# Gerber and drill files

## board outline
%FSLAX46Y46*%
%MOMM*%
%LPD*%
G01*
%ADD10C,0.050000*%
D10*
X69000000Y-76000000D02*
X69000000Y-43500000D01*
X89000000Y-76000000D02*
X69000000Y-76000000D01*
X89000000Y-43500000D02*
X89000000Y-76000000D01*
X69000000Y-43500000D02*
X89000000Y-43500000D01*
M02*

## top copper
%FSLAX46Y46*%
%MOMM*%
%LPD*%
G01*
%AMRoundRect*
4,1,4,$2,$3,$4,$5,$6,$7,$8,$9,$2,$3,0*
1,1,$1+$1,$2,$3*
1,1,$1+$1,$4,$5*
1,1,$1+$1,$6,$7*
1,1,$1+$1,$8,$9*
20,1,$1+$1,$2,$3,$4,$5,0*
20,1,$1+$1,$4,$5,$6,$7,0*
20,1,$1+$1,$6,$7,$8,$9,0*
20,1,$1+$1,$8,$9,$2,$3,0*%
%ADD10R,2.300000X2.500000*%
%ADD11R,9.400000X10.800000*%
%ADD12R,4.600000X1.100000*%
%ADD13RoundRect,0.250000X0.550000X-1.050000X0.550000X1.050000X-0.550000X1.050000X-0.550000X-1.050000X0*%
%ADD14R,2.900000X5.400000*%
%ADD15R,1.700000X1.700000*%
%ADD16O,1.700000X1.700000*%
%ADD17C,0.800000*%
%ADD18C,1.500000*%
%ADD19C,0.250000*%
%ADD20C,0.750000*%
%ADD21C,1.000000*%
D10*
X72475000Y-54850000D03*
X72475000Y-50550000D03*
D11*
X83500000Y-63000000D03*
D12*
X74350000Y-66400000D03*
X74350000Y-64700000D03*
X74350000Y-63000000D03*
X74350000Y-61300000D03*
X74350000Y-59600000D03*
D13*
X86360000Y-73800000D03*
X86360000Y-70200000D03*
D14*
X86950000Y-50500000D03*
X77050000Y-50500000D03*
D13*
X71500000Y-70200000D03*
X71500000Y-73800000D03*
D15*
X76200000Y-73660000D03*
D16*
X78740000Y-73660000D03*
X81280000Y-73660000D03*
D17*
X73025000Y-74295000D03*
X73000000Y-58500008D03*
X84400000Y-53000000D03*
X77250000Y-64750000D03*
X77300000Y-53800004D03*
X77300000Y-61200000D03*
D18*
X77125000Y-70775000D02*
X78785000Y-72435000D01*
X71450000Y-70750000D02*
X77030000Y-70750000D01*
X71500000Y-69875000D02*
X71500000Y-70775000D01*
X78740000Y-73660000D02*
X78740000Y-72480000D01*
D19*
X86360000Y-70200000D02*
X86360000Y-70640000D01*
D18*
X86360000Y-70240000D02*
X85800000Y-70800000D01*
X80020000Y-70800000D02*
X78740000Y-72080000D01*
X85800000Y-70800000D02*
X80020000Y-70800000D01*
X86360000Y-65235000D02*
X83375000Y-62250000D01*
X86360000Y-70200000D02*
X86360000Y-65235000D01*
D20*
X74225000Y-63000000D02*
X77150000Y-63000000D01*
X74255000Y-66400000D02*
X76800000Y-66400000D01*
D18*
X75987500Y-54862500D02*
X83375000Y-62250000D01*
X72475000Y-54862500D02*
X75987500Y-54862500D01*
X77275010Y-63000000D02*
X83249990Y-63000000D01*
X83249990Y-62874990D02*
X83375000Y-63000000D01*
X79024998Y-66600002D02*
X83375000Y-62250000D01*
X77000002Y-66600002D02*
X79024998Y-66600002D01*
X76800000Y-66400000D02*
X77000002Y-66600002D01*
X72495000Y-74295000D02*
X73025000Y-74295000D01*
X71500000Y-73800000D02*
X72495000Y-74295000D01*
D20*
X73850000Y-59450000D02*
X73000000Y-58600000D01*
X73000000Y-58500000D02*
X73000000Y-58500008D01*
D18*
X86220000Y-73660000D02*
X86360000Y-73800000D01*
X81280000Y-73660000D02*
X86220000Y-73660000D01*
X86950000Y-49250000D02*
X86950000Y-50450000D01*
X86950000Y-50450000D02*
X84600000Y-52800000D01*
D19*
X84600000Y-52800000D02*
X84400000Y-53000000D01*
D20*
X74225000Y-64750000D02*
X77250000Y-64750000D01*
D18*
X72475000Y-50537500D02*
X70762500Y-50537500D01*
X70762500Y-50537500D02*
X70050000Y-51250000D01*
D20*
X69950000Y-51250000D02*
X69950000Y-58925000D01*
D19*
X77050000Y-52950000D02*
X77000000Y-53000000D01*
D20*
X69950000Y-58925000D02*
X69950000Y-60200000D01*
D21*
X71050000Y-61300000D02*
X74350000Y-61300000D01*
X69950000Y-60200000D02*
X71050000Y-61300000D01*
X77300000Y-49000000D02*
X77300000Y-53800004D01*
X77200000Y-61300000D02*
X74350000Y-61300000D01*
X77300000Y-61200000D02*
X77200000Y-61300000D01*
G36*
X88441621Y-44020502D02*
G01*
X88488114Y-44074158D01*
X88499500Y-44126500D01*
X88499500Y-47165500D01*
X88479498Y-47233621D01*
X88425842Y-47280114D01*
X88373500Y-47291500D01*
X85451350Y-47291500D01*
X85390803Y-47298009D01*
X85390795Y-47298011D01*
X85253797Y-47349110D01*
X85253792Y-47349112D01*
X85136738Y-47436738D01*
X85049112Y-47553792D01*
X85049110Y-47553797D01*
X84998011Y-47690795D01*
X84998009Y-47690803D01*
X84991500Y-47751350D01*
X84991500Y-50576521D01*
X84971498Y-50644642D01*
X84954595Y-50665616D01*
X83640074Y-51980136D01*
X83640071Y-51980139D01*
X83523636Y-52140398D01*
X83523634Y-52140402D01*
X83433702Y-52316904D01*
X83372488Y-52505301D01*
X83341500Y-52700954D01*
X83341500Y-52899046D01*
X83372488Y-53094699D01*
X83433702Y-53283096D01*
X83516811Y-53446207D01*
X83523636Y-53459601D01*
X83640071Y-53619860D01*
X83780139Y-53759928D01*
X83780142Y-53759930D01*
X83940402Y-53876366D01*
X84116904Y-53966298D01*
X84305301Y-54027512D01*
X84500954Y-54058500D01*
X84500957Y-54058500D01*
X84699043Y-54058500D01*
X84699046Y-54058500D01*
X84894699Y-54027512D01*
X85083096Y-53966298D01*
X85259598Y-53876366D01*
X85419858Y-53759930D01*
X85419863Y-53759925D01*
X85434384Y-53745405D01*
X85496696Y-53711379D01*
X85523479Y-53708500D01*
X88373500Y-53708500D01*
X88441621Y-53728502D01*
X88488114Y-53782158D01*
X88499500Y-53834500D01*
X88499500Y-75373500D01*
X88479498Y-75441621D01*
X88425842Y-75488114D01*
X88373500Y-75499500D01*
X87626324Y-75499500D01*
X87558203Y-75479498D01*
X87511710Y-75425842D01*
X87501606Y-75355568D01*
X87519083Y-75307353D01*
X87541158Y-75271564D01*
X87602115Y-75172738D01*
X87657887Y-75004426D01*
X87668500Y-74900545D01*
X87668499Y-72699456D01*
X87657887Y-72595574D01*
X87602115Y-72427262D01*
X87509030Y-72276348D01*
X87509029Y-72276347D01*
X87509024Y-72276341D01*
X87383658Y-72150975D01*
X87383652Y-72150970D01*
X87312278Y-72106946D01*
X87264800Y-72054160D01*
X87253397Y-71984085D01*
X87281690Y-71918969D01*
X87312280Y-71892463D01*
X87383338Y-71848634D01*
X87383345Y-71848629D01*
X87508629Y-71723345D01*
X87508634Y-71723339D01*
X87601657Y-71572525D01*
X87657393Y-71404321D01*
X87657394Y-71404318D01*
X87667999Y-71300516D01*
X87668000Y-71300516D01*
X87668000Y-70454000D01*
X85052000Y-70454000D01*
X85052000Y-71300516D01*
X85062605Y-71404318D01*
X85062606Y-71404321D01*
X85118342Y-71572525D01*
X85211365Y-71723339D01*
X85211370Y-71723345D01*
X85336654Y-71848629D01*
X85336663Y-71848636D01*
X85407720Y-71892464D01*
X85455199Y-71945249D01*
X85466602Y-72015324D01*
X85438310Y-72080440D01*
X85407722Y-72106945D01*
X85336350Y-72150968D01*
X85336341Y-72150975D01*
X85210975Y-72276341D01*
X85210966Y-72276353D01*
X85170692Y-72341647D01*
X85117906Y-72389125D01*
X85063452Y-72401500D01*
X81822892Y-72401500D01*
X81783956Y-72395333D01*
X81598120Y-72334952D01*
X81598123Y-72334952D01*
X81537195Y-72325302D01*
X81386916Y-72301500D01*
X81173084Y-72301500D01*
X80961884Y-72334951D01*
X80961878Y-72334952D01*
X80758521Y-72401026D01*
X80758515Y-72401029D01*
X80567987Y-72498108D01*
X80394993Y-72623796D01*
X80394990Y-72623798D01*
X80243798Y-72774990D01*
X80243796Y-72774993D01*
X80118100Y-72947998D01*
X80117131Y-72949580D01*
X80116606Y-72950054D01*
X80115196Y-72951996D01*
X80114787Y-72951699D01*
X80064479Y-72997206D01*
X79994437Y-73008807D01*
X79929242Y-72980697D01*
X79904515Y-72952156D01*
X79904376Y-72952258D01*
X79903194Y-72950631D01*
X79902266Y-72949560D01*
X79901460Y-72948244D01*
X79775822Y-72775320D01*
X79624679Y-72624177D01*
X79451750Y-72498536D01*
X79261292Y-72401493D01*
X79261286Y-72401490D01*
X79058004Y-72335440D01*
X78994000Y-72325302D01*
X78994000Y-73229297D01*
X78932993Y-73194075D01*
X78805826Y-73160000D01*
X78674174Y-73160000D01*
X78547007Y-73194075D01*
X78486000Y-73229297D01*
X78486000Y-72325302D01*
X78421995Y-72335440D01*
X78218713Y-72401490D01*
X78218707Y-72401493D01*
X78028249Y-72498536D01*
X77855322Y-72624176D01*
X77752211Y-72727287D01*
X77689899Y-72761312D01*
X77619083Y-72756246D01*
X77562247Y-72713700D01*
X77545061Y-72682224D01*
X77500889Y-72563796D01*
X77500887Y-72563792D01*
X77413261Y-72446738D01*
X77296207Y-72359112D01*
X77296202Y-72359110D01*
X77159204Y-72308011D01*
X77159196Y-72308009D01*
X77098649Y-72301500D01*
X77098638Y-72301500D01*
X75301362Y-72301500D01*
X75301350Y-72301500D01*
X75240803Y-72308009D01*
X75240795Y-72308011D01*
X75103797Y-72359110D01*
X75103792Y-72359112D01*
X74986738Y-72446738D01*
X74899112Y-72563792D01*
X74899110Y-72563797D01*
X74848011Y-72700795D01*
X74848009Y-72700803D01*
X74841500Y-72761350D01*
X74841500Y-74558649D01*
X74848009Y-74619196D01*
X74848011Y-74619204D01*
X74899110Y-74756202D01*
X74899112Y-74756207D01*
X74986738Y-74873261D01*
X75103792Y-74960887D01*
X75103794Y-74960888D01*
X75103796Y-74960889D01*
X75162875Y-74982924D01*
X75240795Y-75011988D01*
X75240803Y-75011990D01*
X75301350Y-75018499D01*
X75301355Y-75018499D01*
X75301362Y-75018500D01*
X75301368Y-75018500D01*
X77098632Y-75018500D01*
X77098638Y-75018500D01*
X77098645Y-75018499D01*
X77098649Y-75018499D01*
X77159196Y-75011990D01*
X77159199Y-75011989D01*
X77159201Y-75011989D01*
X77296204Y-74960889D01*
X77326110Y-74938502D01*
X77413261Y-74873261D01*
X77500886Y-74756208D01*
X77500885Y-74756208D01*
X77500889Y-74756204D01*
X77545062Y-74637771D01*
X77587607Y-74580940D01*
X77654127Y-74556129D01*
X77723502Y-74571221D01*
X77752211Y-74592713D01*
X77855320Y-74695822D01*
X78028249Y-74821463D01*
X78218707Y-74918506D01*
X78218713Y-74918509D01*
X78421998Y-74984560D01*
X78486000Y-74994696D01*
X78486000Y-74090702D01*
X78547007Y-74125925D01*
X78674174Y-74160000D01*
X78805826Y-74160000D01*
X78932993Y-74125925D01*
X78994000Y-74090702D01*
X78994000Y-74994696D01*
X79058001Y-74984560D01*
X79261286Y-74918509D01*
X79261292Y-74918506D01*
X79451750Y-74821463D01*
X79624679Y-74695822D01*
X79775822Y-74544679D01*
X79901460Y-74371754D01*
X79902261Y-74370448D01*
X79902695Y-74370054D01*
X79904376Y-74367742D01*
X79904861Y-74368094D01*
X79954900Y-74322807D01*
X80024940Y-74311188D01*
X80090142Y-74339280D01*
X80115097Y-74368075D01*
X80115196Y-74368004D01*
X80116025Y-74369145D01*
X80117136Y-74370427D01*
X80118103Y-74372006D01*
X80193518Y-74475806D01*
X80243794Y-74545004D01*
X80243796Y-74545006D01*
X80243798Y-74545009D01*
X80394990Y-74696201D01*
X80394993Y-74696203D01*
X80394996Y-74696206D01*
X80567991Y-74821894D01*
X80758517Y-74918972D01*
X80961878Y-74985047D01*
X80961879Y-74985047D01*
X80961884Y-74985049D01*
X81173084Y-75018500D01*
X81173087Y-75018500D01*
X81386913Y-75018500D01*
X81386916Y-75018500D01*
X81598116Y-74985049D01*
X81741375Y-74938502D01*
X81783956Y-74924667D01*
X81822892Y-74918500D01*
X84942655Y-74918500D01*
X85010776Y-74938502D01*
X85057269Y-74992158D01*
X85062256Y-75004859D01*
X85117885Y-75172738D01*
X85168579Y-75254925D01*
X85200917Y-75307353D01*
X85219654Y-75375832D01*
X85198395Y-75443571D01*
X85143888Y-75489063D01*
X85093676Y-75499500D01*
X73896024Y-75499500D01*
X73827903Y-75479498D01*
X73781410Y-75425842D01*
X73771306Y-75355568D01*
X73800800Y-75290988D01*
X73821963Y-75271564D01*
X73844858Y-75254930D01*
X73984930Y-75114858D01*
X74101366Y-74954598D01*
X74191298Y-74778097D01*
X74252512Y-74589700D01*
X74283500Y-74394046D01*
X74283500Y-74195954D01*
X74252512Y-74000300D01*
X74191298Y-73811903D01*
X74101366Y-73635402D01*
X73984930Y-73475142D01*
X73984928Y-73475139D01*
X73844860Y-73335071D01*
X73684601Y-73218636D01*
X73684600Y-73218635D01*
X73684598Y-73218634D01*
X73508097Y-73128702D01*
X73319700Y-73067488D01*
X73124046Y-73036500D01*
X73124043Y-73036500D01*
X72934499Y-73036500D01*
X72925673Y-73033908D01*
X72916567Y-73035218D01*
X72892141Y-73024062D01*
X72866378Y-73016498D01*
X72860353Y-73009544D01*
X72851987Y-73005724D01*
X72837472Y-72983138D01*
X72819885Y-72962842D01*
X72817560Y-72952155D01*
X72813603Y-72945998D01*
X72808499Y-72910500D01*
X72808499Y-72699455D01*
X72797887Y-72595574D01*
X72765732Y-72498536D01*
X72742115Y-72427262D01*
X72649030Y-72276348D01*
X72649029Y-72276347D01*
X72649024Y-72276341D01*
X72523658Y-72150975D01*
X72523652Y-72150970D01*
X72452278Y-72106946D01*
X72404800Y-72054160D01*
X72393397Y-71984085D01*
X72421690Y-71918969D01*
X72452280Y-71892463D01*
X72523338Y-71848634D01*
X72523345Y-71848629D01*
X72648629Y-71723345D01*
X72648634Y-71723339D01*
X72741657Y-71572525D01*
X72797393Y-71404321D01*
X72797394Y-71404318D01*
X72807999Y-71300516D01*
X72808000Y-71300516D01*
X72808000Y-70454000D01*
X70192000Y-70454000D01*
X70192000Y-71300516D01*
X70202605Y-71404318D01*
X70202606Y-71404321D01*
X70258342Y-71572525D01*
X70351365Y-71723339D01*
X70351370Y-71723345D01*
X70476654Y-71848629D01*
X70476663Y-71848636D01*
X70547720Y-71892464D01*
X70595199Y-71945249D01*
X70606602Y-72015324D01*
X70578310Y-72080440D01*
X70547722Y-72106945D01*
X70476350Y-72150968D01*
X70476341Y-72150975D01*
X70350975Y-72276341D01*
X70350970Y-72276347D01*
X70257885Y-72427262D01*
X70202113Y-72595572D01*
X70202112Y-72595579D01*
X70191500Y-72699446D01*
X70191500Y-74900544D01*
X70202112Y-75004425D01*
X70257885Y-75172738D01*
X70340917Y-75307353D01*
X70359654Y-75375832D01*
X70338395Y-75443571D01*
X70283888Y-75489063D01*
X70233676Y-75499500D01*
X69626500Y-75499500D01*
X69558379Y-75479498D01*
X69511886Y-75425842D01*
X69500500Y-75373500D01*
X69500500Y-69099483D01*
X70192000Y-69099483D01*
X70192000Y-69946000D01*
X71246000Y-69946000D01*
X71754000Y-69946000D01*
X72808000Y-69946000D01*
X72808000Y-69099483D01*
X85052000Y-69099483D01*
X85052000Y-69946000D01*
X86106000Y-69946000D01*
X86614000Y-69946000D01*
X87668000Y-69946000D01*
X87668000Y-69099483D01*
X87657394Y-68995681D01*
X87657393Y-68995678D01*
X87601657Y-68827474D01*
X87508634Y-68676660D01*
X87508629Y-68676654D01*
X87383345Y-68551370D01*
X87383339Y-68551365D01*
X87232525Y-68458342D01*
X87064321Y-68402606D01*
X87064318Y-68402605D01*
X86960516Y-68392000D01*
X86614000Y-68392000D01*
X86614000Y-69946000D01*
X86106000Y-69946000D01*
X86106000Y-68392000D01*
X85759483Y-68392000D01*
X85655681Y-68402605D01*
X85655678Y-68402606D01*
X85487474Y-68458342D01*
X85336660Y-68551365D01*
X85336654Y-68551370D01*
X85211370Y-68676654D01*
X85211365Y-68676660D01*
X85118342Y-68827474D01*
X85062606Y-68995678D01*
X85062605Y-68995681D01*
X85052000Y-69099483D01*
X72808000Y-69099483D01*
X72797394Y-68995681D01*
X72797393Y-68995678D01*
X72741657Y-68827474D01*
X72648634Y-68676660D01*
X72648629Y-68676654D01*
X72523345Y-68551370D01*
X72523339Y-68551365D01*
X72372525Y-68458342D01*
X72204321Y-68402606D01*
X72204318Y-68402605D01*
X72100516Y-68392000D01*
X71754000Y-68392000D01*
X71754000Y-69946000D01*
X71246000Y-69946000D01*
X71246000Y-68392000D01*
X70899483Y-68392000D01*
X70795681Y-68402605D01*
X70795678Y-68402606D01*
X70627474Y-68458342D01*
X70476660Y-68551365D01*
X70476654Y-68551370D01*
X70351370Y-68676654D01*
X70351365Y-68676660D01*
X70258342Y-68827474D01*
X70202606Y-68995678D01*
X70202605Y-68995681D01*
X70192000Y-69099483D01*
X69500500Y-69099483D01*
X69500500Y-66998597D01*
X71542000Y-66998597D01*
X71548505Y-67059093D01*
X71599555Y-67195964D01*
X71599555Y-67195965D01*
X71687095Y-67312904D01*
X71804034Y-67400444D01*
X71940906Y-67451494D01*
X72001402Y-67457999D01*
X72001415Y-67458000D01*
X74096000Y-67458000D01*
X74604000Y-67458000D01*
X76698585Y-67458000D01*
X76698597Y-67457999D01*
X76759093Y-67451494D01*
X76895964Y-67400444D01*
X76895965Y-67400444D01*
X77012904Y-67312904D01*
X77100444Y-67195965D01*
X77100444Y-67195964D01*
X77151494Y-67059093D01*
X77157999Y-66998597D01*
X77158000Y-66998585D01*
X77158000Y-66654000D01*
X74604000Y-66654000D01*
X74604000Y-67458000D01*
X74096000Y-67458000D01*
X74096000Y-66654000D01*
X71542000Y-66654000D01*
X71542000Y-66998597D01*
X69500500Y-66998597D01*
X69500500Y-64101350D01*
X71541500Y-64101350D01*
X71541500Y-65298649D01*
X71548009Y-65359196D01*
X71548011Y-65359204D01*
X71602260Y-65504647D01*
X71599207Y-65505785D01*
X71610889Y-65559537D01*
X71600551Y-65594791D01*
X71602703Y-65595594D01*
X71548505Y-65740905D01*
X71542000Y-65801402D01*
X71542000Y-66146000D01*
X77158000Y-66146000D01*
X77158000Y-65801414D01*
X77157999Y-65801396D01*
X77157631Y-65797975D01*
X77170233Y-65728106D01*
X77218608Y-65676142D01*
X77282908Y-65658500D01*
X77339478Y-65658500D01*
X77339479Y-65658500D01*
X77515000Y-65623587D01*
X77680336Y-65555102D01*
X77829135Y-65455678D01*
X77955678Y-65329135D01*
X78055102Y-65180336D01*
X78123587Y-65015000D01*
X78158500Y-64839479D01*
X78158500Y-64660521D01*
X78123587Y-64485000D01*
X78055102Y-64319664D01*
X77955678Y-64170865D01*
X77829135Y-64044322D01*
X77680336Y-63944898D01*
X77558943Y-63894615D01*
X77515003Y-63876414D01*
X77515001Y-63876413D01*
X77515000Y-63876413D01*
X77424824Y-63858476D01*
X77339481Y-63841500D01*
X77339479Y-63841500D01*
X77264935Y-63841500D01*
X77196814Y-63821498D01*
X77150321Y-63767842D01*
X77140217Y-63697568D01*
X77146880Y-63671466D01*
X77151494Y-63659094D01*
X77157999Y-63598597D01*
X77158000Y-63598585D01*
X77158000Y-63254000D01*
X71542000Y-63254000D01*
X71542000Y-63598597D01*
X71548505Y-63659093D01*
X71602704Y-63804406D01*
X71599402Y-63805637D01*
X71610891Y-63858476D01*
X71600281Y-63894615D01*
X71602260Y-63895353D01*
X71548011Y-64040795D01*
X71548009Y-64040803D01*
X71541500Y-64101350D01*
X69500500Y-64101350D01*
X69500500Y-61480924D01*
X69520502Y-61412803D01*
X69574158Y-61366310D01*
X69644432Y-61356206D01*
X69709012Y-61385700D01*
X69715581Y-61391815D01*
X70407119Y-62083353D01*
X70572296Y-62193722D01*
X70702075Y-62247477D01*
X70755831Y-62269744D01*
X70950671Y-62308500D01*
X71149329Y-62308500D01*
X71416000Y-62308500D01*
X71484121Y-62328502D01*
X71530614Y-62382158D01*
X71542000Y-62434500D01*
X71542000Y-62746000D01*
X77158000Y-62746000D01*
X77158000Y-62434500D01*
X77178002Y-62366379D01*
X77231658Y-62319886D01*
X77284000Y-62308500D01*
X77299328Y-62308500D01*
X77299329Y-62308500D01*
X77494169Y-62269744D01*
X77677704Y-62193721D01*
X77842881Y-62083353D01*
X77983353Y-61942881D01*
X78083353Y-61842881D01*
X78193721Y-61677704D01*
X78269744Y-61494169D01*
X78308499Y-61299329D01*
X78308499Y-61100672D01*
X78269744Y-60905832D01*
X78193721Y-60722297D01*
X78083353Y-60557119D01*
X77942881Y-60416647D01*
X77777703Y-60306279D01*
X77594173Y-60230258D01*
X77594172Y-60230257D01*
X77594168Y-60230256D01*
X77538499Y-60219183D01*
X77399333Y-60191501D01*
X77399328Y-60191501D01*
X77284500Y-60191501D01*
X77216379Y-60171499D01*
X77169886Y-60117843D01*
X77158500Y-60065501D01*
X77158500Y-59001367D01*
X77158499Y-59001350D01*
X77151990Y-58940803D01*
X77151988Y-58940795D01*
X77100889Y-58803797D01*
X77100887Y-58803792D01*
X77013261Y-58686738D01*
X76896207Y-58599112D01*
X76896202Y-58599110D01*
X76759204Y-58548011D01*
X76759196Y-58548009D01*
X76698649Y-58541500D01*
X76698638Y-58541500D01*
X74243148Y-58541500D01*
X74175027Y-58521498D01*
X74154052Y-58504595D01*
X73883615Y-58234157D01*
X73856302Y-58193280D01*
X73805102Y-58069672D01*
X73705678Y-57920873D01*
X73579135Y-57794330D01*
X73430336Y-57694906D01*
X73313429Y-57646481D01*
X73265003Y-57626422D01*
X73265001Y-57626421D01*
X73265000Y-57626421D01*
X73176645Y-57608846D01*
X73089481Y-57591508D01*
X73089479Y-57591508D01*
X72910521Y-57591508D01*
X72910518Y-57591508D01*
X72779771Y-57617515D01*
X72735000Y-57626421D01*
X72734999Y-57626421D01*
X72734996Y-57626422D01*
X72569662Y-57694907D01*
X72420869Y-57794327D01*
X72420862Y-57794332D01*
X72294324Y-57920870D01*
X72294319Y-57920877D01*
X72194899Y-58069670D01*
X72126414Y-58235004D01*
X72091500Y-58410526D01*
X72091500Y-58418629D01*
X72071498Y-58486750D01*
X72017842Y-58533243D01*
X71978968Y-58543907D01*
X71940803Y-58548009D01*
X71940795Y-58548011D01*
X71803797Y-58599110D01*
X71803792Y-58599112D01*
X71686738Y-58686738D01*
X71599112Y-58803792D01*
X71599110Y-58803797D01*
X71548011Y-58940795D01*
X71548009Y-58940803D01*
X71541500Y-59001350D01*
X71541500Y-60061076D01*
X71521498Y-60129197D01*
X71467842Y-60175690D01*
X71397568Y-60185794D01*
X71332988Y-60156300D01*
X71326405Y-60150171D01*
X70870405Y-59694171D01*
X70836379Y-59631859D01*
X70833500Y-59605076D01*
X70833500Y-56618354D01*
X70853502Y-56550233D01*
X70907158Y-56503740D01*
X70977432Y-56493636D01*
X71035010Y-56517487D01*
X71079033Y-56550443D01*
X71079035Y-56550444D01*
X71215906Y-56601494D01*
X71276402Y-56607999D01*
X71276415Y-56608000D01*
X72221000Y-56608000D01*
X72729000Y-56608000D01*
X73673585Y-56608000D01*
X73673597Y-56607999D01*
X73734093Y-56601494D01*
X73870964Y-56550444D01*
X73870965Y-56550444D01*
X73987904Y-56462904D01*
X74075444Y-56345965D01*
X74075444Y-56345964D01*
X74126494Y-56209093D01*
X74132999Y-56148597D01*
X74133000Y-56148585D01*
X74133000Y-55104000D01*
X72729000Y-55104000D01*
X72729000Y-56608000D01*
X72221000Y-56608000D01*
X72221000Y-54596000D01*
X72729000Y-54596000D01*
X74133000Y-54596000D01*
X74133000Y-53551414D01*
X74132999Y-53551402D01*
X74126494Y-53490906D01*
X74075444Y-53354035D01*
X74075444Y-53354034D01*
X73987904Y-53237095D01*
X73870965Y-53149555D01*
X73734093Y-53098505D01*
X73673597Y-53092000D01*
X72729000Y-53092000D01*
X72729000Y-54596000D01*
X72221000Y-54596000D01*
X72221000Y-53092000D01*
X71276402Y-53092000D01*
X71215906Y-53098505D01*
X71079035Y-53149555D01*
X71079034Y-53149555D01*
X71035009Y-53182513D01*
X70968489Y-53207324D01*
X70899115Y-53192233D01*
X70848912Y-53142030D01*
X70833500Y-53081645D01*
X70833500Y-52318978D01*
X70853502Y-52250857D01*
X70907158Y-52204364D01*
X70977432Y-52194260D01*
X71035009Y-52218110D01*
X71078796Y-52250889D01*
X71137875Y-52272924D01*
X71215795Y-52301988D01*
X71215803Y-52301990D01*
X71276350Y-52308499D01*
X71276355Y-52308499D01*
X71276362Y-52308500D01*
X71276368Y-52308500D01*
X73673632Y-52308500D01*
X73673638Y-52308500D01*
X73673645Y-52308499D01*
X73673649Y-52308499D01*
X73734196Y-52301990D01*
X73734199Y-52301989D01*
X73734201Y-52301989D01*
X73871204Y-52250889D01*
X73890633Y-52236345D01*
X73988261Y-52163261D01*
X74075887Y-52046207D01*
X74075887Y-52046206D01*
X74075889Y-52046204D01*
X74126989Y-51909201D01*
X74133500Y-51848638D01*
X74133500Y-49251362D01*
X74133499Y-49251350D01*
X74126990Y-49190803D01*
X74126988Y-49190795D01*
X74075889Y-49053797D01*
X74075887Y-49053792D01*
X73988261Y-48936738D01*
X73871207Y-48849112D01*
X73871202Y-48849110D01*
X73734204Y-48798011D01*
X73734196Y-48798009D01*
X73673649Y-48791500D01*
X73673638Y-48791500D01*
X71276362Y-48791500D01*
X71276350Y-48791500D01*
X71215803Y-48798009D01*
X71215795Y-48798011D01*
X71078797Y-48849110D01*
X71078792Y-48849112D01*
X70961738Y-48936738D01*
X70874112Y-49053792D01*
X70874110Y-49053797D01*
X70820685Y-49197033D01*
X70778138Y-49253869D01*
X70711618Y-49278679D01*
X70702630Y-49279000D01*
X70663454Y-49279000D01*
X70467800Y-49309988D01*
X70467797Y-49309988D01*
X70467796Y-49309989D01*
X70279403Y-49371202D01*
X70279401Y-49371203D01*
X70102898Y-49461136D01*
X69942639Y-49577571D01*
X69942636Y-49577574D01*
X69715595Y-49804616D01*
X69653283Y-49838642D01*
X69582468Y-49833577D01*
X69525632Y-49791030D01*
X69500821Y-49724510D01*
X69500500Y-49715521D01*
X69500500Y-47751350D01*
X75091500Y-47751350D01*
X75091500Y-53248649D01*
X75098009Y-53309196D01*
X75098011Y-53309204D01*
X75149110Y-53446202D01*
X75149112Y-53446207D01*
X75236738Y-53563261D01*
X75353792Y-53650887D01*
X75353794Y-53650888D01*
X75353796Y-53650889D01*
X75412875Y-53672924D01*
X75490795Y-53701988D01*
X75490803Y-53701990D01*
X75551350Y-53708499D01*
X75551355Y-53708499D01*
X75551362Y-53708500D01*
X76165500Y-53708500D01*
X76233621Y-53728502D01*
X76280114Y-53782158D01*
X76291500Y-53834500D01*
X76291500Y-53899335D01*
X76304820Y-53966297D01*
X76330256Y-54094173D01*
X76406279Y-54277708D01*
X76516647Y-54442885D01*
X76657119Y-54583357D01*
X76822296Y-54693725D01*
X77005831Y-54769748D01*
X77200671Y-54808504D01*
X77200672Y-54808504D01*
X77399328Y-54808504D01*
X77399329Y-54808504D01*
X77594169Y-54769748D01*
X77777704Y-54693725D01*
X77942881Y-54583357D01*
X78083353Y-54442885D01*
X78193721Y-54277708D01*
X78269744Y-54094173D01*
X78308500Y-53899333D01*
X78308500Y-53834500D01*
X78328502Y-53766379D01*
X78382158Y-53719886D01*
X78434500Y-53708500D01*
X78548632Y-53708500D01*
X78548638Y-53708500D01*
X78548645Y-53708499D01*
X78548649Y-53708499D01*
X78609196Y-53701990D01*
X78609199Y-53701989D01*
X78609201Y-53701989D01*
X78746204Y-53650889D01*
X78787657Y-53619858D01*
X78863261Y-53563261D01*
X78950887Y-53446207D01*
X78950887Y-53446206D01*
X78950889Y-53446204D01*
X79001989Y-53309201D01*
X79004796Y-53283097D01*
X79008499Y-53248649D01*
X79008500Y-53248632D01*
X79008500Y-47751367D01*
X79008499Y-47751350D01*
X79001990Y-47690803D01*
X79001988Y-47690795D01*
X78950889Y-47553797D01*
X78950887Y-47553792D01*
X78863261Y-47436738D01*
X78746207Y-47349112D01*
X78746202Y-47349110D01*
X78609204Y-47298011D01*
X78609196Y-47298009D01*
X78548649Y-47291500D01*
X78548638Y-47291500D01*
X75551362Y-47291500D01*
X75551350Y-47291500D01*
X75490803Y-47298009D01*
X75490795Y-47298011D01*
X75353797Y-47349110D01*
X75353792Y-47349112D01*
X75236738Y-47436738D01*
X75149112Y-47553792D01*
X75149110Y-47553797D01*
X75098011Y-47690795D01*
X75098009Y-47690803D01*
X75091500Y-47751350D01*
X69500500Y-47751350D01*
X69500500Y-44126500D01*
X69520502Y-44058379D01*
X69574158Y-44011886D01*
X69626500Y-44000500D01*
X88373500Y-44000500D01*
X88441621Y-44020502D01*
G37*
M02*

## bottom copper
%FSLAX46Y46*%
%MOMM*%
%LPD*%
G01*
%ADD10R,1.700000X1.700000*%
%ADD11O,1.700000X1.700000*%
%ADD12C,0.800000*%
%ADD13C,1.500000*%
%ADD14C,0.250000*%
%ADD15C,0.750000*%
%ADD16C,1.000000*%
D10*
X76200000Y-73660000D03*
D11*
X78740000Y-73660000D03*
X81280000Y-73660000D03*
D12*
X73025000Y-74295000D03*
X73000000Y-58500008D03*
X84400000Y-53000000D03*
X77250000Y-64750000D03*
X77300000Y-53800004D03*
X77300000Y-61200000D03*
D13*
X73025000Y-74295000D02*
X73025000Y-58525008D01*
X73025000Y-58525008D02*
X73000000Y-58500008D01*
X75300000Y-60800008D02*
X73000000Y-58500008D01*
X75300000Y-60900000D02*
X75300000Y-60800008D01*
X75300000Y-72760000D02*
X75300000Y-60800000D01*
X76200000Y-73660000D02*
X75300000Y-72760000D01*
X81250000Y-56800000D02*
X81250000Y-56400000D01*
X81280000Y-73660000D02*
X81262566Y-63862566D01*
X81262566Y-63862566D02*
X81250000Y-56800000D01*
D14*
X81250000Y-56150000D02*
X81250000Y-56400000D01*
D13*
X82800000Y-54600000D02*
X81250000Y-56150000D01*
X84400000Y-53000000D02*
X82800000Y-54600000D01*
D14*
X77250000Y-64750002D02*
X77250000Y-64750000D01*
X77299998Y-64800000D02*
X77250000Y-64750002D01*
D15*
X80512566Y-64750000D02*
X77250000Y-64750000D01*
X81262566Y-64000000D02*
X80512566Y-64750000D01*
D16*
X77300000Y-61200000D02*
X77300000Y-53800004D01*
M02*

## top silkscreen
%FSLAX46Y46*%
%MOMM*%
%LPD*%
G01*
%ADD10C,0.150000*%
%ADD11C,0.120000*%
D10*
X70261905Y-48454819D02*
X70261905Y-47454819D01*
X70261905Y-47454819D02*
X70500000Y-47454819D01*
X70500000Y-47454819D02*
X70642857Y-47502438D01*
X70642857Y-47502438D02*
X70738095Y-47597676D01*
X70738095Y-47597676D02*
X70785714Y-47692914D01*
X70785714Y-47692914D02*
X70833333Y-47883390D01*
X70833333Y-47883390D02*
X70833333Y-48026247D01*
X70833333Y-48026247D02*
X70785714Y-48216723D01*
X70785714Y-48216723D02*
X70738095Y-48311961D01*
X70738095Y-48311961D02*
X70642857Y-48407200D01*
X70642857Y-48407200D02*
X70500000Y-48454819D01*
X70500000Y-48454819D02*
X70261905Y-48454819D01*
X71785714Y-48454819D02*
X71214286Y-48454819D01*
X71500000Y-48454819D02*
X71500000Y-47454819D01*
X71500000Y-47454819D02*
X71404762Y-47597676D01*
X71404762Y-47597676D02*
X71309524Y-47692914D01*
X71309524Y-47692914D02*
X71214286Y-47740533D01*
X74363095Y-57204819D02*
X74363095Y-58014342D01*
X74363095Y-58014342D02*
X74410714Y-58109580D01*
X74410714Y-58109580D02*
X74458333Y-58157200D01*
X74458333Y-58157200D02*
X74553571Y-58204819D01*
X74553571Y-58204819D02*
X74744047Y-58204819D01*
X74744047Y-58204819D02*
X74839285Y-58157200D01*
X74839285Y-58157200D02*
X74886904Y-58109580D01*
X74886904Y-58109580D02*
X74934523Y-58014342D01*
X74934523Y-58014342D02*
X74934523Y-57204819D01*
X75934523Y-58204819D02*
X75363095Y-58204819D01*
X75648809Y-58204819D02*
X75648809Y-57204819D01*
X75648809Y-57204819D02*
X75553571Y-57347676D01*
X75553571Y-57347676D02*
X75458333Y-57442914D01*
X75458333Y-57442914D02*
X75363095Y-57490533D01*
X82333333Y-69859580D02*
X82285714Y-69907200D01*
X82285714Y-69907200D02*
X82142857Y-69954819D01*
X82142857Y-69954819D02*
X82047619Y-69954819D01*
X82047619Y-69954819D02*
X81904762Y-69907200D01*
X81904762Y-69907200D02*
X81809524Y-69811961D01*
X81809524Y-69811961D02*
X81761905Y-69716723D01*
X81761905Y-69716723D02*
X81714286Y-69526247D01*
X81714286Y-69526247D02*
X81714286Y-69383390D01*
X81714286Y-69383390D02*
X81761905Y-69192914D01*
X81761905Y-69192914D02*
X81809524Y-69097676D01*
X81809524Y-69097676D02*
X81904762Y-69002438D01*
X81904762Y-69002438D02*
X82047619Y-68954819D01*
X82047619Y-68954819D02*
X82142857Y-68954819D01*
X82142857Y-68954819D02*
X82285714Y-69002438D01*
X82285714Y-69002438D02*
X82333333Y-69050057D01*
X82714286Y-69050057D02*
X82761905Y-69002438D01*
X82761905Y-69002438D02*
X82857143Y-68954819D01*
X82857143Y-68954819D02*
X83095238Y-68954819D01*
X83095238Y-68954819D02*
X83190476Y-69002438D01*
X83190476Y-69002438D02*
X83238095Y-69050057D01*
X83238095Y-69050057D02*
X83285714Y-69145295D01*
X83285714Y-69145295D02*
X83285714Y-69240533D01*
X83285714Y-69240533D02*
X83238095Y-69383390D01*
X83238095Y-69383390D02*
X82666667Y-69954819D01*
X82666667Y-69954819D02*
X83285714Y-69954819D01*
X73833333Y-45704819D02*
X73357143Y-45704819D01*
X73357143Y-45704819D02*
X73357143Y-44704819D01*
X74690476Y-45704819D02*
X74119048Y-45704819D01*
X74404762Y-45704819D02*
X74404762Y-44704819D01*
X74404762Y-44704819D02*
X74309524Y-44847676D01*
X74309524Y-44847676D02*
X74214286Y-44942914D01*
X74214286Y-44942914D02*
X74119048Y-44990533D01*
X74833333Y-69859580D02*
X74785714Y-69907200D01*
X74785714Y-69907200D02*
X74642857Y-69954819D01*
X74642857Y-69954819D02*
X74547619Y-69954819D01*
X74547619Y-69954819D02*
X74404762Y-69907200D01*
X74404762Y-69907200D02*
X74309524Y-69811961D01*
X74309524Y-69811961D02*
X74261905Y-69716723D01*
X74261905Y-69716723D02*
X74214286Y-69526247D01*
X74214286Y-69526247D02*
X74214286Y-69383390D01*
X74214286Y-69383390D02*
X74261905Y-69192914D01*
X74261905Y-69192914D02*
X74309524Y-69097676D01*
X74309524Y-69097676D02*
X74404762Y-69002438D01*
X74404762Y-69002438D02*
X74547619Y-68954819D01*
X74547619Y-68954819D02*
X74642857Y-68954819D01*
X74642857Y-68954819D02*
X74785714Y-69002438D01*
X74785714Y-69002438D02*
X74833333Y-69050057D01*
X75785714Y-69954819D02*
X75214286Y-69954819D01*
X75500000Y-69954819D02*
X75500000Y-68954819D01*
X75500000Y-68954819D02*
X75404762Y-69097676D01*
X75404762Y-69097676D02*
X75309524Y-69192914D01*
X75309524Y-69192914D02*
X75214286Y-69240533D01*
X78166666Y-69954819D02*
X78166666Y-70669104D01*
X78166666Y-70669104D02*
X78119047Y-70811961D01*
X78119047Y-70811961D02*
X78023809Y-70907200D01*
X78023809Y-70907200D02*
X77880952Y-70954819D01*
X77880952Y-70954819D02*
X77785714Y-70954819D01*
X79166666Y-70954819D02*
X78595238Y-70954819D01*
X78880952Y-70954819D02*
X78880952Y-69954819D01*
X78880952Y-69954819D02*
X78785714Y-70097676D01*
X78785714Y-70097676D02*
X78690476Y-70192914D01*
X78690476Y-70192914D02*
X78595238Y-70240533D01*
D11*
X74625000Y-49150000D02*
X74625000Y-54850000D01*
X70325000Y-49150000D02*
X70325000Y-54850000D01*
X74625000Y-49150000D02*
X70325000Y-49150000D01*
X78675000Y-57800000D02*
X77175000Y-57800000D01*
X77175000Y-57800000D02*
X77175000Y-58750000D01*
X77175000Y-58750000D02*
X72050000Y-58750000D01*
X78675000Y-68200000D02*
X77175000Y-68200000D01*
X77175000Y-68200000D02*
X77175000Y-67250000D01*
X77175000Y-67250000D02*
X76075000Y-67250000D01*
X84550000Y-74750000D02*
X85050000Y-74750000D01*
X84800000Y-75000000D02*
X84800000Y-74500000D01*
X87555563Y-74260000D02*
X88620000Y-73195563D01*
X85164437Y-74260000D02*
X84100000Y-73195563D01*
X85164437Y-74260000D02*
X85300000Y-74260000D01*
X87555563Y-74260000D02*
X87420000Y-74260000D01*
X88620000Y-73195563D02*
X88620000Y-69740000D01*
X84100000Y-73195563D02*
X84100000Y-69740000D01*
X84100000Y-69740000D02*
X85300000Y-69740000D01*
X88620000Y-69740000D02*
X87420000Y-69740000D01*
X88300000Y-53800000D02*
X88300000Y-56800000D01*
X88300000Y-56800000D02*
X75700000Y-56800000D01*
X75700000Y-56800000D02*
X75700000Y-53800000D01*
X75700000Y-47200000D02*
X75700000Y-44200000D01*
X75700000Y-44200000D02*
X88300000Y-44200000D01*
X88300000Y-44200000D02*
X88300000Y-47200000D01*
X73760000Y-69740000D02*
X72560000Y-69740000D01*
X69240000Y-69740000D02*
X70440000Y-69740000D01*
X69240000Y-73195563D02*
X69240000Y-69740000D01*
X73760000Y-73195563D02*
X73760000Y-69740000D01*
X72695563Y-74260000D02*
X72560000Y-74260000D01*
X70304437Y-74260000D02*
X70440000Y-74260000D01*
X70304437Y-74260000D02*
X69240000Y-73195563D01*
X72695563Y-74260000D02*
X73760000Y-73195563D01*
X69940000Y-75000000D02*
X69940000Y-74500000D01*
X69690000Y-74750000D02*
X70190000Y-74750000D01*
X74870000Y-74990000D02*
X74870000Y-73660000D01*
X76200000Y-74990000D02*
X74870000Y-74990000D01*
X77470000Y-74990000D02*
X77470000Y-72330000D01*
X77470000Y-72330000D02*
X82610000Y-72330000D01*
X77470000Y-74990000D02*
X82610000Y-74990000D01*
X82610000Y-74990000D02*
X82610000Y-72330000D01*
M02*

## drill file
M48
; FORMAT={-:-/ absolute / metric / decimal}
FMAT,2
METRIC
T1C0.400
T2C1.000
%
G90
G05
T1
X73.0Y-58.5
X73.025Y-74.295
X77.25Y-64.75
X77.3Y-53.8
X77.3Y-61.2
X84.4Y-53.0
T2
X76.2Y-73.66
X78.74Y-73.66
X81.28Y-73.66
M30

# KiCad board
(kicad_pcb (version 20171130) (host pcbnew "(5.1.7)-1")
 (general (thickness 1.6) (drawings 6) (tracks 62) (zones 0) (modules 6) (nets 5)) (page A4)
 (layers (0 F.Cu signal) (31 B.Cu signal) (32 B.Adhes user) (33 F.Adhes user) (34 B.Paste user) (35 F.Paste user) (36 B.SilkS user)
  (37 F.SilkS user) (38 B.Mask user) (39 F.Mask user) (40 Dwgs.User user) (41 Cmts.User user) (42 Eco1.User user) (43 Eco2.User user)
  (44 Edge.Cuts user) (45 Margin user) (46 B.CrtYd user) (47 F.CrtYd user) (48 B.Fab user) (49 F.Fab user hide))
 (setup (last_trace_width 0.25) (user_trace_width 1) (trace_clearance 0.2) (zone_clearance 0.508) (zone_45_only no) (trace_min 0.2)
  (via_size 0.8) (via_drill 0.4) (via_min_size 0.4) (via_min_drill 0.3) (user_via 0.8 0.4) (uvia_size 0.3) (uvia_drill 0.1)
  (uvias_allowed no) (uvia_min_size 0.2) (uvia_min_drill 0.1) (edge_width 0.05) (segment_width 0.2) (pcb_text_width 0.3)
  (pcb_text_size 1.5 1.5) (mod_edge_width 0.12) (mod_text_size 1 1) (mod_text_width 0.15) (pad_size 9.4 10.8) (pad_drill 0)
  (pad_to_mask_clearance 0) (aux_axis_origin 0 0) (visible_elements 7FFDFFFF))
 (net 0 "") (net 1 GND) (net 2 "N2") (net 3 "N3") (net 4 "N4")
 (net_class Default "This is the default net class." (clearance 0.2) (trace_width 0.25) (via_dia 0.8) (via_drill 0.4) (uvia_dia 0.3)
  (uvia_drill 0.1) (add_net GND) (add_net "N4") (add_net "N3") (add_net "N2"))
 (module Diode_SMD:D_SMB (layer F.Cu) (at 72.475 52.7 270)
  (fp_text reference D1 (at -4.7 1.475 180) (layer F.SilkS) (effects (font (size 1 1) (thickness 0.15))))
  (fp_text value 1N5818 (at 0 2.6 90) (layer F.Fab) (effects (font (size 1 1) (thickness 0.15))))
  (fp_line (start -3.55 -2.15) (end 2.15 -2.15) (layer F.SilkS) (width 0.12))
  (fp_line (start -3.55 2.15) (end 2.15 2.15) (layer F.SilkS) (width 0.12))
  (fp_line (start -3.55 -2.15) (end -3.55 2.15) (layer F.SilkS) (width 0.12))
  (pad 2 smd rect (at 2.15 0 270) (size 2.5 2.3) (layers F.Cu F.Paste F.Mask) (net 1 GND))
  (pad 1 smd rect (at -2.15 0 270) (size 2.5 2.3) (layers F.Cu F.Paste F.Mask) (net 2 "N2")))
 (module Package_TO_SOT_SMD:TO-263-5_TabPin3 (layer F.Cu) (at 80.125 63)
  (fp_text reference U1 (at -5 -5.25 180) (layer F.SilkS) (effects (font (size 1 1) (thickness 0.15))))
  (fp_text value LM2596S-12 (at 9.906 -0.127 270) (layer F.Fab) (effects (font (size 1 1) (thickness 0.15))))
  (fp_line (start -1.45 -5.2) (end -2.95 -5.2) (layer F.SilkS) (width 0.12))
  (fp_line (start -2.95 -5.2) (end -2.95 -4.25) (layer F.SilkS) (width 0.12))
  (fp_line (start -2.95 -4.25) (end -8.075 -4.25) (layer F.SilkS) (width 0.12))
  (fp_line (start -1.45 5.2) (end -2.95 5.2) (layer F.SilkS) (width 0.12))
  (fp_line (start -2.95 5.2) (end -2.95 4.25) (layer F.SilkS) (width 0.12))
  (fp_line (start -2.95 4.25) (end -4.05 4.25) (layer F.SilkS) (width 0.12))
  (pad "" smd rect (at 0.95 2.775) (size 4.55 5.25) (layers F.Paste))
  (pad "" smd rect (at 5.8 -2.775) (size 4.55 5.25) (layers F.Paste))
  (pad "" smd rect (at 0.95 -2.775) (size 4.55 5.25) (layers F.Paste))
  (pad "" smd rect (at 5.8 2.775) (size 4.55 5.25) (layers F.Paste))
  (pad 3 smd rect (at 3.375 0) (size 9.4 10.8) (layers F.Cu F.Mask) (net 1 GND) (zone_connect 2))
  (pad 5 smd rect (at -5.775 3.4) (size 4.6 1.1) (layers F.Cu F.Paste F.Mask) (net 1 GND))
  (pad FEDBACK smd rect (at -5.775 1.7) (size 4.6 1.1) (layers F.Cu F.Paste F.Mask) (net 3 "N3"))
  (pad 3 smd rect (at -5.775 0) (size 4.6 1.1) (layers F.Cu F.Paste F.Mask) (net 1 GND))
  (pad OUTPUT smd rect (at -5.775 -1.7) (size 4.6 1.1) (layers F.Cu F.Paste F.Mask) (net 2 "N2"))
  (pad INPUT smd rect (at -5.775 -3.4) (size 4.6 1.1) (layers F.Cu F.Paste F.Mask) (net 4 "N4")))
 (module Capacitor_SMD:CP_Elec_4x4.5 (layer F.Cu) (at 86.36 72 90)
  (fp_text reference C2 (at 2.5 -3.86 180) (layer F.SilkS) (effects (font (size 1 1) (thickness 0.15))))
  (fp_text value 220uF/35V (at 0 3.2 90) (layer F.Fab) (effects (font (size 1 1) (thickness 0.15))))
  (fp_line (start -2.75 -1.81) (end -2.75 -1.31) (layer F.SilkS) (width 0.12))
  (fp_line (start -3 -1.56) (end -2.5 -1.56) (layer F.SilkS) (width 0.12))
  (fp_line (start -2.26 1.195563) (end -1.195563 2.26) (layer F.SilkS) (width 0.12))
  (fp_line (start -2.26 -1.195563) (end -1.195563 -2.26) (layer F.SilkS) (width 0.12))
  (fp_line (start -2.26 -1.195563) (end -2.26 -1.06) (layer F.SilkS) (width 0.12))
  (fp_line (start -2.26 1.195563) (end -2.26 1.06) (layer F.SilkS) (width 0.12))
  (fp_line (start -1.195563 2.26) (end 2.26 2.26) (layer F.SilkS) (width 0.12))
  (fp_line (start -1.195563 -2.26) (end 2.26 -2.26) (layer F.SilkS) (width 0.12))
  (fp_line (start 2.26 -2.26) (end 2.26 -1.06) (layer F.SilkS) (width 0.12))
  (fp_line (start 2.26 2.26) (end 2.26 1.06) (layer F.SilkS) (width 0.12))
  (pad 1 smd roundrect (at -1.8 0 90) (size 2.6 1.6) (layers F.Cu F.Paste F.Mask) (roundrect_rratio 0.15625) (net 3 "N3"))
  (pad 2 smd roundrect (at 1.8 0 90) (size 2.6 1.6) (layers F.Cu F.Paste F.Mask) (roundrect_rratio 0.15625) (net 1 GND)))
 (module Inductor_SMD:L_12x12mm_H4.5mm (layer F.Cu) (at 82 50.5)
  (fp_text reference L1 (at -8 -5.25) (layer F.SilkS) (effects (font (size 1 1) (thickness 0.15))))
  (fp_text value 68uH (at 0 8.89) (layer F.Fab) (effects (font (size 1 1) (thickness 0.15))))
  (fp_line (start 6.3 3.3) (end 6.3 6.3) (layer F.SilkS) (width 0.12))
  (fp_line (start 6.3 6.3) (end -6.3 6.3) (layer F.SilkS) (width 0.12))
  (fp_line (start -6.3 6.3) (end -6.3 3.3) (layer F.SilkS) (width 0.12))
  (fp_line (start -6.3 -3.3) (end -6.3 -6.3) (layer F.SilkS) (width 0.12))
  (fp_line (start -6.3 -6.3) (end 6.3 -6.3) (layer F.SilkS) (width 0.12))
  (fp_line (start 6.3 -6.3) (end 6.3 -3.3) (layer F.SilkS) (width 0.12))
  (pad 2 smd rect (at 4.95 0) (size 2.9 5.4) (layers F.Cu F.Paste F.Mask) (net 3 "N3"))
  (pad 1 smd rect (at -4.95 0) (size 2.9 5.4) (layers F.Cu F.Paste F.Mask) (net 2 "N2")))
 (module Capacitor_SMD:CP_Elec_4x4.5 (layer F.Cu) (at 71.5 72 90)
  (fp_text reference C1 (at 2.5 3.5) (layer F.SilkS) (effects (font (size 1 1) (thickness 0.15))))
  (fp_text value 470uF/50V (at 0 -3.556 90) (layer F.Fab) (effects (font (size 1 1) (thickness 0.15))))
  (fp_line (start 2.26 2.26) (end 2.26 1.06) (layer F.SilkS) (width 0.12))
  (fp_line (start 2.26 -2.26) (end 2.26 -1.06) (layer F.SilkS) (width 0.12))
  (fp_line (start -1.195563 -2.26) (end 2.26 -2.26) (layer F.SilkS) (width 0.12))
  (fp_line (start -1.195563 2.26) (end 2.26 2.26) (layer F.SilkS) (width 0.12))
  (fp_line (start -2.26 1.195563) (end -2.26 1.06) (layer F.SilkS) (width 0.12))
  (fp_line (start -2.26 -1.195563) (end -2.26 -1.06) (layer F.SilkS) (width 0.12))
  (fp_line (start -2.26 -1.195563) (end -1.195563 -2.26) (layer F.SilkS) (width 0.12))
  (fp_line (start -2.26 1.195563) (end -1.195563 2.26) (layer F.SilkS) (width 0.12))
  (fp_line (start -3 -1.56) (end -2.5 -1.56) (layer F.SilkS) (width 0.12))
  (fp_line (start -2.75 -1.81) (end -2.75 -1.31) (layer F.SilkS) (width 0.12))
  (pad 2 smd roundrect (at 1.8 0 90) (size 2.6 1.6) (layers F.Cu F.Paste F.Mask) (roundrect_rratio 0.15625) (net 1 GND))
  (pad 1 smd roundrect (at -1.8 0 90) (size 2.6 1.6) (layers F.Cu F.Paste F.Mask) (roundrect_rratio 0.15625) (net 4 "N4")))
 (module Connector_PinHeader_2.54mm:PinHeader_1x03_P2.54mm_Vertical (layer F.Cu) (at 76.2 73.66 90)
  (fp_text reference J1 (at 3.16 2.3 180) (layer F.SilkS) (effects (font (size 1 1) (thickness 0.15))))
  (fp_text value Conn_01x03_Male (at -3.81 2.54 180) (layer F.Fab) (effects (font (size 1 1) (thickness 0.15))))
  (fp_line (start -1.33 -1.33) (end 0 -1.33) (layer F.SilkS) (width 0.12))
  (fp_line (start -1.33 0) (end -1.33 -1.33) (layer F.SilkS) (width 0.12))
  (fp_line (start -1.33 1.27) (end 1.33 1.27) (layer F.SilkS) (width 0.12))
  (fp_line (start 1.33 1.27) (end 1.33 6.41) (layer F.SilkS) (width 0.12))
  (fp_line (start -1.33 1.27) (end -1.33 6.41) (layer F.SilkS) (width 0.12))
  (fp_line (start -1.33 6.41) (end 1.33 6.41) (layer F.SilkS) (width 0.12))
  (pad 1 thru_hole rect (at 0 0 90) (size 1.7 1.7) (drill 1) (layers *.Cu *.Mask) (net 4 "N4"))
  (pad 2 thru_hole oval (at 0 2.54 90) (size 1.7 1.7) (drill 1) (layers *.Cu *.Mask) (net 1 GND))
  (pad 3 thru_hole oval (at 0 5.08 90) (size 1.7 1.7) (drill 1) (layers *.Cu *.Mask) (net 3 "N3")))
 (gr_line (start 69 76) (end 69 43.5) (layer Edge.Cuts) (width 0.05))
 (gr_line (start 89 76) (end 69 76) (layer Edge.Cuts) (width 0.05))
 (gr_line (start 89 43.5) (end 89 76) (layer Edge.Cuts) (width 0.05))
 (gr_line (start 69 43.5) (end 89 43.5) (layer Edge.Cuts) (width 0.05))
 (segment (start 77.125 70.775) (end 78.785 72.435) (width 1.5) (layer F.Cu) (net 1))
 (segment (start 71.45 70.75) (end 77.03 70.75) (width 1.5) (layer F.Cu) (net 1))
 (segment (start 71.5 69.875) (end 71.5 70.775) (width 1.5) (layer F.Cu) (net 1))
 (segment (start 78.74 73.66) (end 78.74 72.48) (width 1.5) (layer F.Cu) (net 1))
 (segment (start 86.36 70.2) (end 86.36 70.64) (width 0.25) (layer F.Cu) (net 1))
 (segment (start 86.36 70.24) (end 85.8 70.8) (width 1.5) (layer F.Cu) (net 1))
 (segment (start 80.02 70.8) (end 78.74 72.08) (width 1.5) (layer F.Cu) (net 1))
 (segment (start 85.8 70.8) (end 80.02 70.8) (width 1.5) (layer F.Cu) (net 1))
 (segment (start 86.36 65.235) (end 83.375 62.25) (width 1.5) (layer F.Cu) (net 1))
 (segment (start 86.36 70.2) (end 86.36 65.235) (width 1.5) (layer F.Cu) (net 1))
 (segment (start 74.225 63) (end 77.15 63) (width 0.75) (layer F.Cu) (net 1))
 (segment (start 74.255 66.4) (end 76.8 66.4) (width 0.75) (layer F.Cu) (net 1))
 (segment (start 75.9875 54.8625) (end 83.375 62.25) (width 1.5) (layer F.Cu) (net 1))
 (segment (start 72.475 54.8625) (end 75.9875 54.8625) (width 1.5) (layer F.Cu) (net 1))
 (segment (start 77.27501 63) (end 83.24999 63) (width 1.5) (layer F.Cu) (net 1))
 (segment (start 83.24999 62.87499) (end 83.375 63) (width 1.5) (layer F.Cu) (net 1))
 (segment (start 79.024998 66.600002) (end 83.375 62.25) (width 1.5) (layer F.Cu) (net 1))
 (segment (start 77.000002 66.600002) (end 79.024998 66.600002) (width 1.5) (layer F.Cu) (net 1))
 (segment (start 76.8 66.4) (end 77.000002 66.600002) (width 1.5) (layer F.Cu) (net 1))
 (via (at 73.025 74.295) (size 0.8) (drill 0.4) (layers F.Cu B.Cu) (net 4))
 (segment (start 72.495 74.295) (end 73.025 74.295) (width 1.5) (layer F.Cu) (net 4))
 (segment (start 71.5 73.8) (end 72.495 74.295) (width 1.5) (layer F.Cu) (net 4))
 (segment (start 73.85 59.45) (end 73 58.6) (width 0.75) (layer F.Cu) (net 4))
 (via (at 73 58.500008) (size 0.8) (drill 0.4) (layers F.Cu B.Cu) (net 4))
 (segment (start 73 58.5) (end 73 58.500008) (width 0.75) (layer F.Cu) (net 4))
 (segment (start 73.025 74.295) (end 73.025 58.525008) (width 1.5) (layer B.Cu) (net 4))
 (segment (start 73.025 58.525008) (end 73 58.500008) (width 1.5) (layer B.Cu) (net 4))
 (segment (start 75.3 60.800008) (end 73 58.500008) (width 1.5) (layer B.Cu) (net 4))
 (segment (start 75.3 60.9) (end 75.3 60.800008) (width 1.5) (layer B.Cu) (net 4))
 (segment (start 75.3 72.76) (end 75.3 60.8) (width 1.5) (layer B.Cu) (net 4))
 (segment (start 76.2 73.66) (end 75.3 72.76) (width 1.5) (layer B.Cu) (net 4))
 (segment (start 86.22 73.66) (end 86.36 73.8) (width 1.5) (layer F.Cu) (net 3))
 (segment (start 81.28 73.66) (end 86.22 73.66) (width 1.5) (layer F.Cu) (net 3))
 (segment (start 81.25 56.8) (end 81.25 56.4) (width 1.5) (layer B.Cu) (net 3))
 (segment (start 81.28 73.66) (end 81.262566 63.862566) (width 1.5) (layer B.Cu) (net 3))
 (segment (start 81.262566 63.862566) (end 81.25 56.8) (width 1.5) (layer B.Cu) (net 3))
 (segment (start 86.95 49.25) (end 86.95 50.45) (width 1.5) (layer F.Cu) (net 3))
 (segment (start 86.95 50.45) (end 84.6 52.8) (width 1.5) (layer F.Cu) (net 3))
 (via (at 84.4 53) (size 0.8) (drill 0.4) (layers F.Cu B.Cu) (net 3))
 (segment (start 84.6 52.8) (end 84.4 53) (width 0.25) (layer F.Cu) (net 3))
 (segment (start 81.25 56.15) (end 81.25 56.4) (width 0.25) (layer B.Cu) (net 3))
 (segment (start 82.8 54.6) (end 81.25 56.15) (width 1.5) (layer B.Cu) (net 3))
 (segment (start 84.4 53) (end 82.8 54.6) (width 1.5) (layer B.Cu) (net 3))
 (segment (start 77.25 64.750002) (end 77.25 64.75) (width 0.25) (layer B.Cu) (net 3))
 (segment (start 77.299998 64.8) (end 77.25 64.750002) (width 0.25) (layer B.Cu) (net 3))
 (segment (start 80.512566 64.75) (end 77.25 64.75) (width 0.75) (layer B.Cu) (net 3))
 (segment (start 81.262566 64) (end 80.512566 64.75) (width 0.75) (layer B.Cu) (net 3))
 (segment (start 74.225 64.75) (end 77.25 64.75) (width 0.75) (layer F.Cu) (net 3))
 (via (at 77.25 64.75) (size 0.8) (drill 0.4) (layers F.Cu B.Cu) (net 3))
 (segment (start 72.475 50.5375) (end 70.7625 50.5375) (width 1.5) (layer F.Cu) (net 2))
 (segment (start 70.7625 50.5375) (end 70.05 51.25) (width 1.5) (layer F.Cu) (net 2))
 (segment (start 69.95 51.25) (end 69.95 58.925) (width 0.75) (layer F.Cu) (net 2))
 (segment (start 77.05 52.95) (end 77 53) (width 0.25) (layer F.Cu) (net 2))
 (segment (start 69.95 58.925) (end 69.95 60.2) (width 0.75) (layer F.Cu) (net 2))
 (segment (start 71.05 61.3) (end 74.35 61.3) (width 1) (layer F.Cu) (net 2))
 (segment (start 69.95 60.2) (end 71.05 61.3) (width 1) (layer F.Cu) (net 2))
 (via (at 77.3 53.800004) (size 0.8) (drill 0.4) (layers F.Cu B.Cu) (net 2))
 (segment (start 77.3 49) (end 77.3 53.800004) (width 1) (layer F.Cu) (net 2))
 (via (at 77.3 61.2) (size 0.8) (drill 0.4) (layers F.Cu B.Cu) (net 2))
 (segment (start 77.2 61.3) (end 74.35 61.3) (width 1) (layer F.Cu) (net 2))
 (segment (start 77.3 61.2) (end 77.2 61.3) (width 1) (layer F.Cu) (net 2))
 (segment (start 77.3 61.2) (end 77.3 53.800004) (width 1) (layer B.Cu) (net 2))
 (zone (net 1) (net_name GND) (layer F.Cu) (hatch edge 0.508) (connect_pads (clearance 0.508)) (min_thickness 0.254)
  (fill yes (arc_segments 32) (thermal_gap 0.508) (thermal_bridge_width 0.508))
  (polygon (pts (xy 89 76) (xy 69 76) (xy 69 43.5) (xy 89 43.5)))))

